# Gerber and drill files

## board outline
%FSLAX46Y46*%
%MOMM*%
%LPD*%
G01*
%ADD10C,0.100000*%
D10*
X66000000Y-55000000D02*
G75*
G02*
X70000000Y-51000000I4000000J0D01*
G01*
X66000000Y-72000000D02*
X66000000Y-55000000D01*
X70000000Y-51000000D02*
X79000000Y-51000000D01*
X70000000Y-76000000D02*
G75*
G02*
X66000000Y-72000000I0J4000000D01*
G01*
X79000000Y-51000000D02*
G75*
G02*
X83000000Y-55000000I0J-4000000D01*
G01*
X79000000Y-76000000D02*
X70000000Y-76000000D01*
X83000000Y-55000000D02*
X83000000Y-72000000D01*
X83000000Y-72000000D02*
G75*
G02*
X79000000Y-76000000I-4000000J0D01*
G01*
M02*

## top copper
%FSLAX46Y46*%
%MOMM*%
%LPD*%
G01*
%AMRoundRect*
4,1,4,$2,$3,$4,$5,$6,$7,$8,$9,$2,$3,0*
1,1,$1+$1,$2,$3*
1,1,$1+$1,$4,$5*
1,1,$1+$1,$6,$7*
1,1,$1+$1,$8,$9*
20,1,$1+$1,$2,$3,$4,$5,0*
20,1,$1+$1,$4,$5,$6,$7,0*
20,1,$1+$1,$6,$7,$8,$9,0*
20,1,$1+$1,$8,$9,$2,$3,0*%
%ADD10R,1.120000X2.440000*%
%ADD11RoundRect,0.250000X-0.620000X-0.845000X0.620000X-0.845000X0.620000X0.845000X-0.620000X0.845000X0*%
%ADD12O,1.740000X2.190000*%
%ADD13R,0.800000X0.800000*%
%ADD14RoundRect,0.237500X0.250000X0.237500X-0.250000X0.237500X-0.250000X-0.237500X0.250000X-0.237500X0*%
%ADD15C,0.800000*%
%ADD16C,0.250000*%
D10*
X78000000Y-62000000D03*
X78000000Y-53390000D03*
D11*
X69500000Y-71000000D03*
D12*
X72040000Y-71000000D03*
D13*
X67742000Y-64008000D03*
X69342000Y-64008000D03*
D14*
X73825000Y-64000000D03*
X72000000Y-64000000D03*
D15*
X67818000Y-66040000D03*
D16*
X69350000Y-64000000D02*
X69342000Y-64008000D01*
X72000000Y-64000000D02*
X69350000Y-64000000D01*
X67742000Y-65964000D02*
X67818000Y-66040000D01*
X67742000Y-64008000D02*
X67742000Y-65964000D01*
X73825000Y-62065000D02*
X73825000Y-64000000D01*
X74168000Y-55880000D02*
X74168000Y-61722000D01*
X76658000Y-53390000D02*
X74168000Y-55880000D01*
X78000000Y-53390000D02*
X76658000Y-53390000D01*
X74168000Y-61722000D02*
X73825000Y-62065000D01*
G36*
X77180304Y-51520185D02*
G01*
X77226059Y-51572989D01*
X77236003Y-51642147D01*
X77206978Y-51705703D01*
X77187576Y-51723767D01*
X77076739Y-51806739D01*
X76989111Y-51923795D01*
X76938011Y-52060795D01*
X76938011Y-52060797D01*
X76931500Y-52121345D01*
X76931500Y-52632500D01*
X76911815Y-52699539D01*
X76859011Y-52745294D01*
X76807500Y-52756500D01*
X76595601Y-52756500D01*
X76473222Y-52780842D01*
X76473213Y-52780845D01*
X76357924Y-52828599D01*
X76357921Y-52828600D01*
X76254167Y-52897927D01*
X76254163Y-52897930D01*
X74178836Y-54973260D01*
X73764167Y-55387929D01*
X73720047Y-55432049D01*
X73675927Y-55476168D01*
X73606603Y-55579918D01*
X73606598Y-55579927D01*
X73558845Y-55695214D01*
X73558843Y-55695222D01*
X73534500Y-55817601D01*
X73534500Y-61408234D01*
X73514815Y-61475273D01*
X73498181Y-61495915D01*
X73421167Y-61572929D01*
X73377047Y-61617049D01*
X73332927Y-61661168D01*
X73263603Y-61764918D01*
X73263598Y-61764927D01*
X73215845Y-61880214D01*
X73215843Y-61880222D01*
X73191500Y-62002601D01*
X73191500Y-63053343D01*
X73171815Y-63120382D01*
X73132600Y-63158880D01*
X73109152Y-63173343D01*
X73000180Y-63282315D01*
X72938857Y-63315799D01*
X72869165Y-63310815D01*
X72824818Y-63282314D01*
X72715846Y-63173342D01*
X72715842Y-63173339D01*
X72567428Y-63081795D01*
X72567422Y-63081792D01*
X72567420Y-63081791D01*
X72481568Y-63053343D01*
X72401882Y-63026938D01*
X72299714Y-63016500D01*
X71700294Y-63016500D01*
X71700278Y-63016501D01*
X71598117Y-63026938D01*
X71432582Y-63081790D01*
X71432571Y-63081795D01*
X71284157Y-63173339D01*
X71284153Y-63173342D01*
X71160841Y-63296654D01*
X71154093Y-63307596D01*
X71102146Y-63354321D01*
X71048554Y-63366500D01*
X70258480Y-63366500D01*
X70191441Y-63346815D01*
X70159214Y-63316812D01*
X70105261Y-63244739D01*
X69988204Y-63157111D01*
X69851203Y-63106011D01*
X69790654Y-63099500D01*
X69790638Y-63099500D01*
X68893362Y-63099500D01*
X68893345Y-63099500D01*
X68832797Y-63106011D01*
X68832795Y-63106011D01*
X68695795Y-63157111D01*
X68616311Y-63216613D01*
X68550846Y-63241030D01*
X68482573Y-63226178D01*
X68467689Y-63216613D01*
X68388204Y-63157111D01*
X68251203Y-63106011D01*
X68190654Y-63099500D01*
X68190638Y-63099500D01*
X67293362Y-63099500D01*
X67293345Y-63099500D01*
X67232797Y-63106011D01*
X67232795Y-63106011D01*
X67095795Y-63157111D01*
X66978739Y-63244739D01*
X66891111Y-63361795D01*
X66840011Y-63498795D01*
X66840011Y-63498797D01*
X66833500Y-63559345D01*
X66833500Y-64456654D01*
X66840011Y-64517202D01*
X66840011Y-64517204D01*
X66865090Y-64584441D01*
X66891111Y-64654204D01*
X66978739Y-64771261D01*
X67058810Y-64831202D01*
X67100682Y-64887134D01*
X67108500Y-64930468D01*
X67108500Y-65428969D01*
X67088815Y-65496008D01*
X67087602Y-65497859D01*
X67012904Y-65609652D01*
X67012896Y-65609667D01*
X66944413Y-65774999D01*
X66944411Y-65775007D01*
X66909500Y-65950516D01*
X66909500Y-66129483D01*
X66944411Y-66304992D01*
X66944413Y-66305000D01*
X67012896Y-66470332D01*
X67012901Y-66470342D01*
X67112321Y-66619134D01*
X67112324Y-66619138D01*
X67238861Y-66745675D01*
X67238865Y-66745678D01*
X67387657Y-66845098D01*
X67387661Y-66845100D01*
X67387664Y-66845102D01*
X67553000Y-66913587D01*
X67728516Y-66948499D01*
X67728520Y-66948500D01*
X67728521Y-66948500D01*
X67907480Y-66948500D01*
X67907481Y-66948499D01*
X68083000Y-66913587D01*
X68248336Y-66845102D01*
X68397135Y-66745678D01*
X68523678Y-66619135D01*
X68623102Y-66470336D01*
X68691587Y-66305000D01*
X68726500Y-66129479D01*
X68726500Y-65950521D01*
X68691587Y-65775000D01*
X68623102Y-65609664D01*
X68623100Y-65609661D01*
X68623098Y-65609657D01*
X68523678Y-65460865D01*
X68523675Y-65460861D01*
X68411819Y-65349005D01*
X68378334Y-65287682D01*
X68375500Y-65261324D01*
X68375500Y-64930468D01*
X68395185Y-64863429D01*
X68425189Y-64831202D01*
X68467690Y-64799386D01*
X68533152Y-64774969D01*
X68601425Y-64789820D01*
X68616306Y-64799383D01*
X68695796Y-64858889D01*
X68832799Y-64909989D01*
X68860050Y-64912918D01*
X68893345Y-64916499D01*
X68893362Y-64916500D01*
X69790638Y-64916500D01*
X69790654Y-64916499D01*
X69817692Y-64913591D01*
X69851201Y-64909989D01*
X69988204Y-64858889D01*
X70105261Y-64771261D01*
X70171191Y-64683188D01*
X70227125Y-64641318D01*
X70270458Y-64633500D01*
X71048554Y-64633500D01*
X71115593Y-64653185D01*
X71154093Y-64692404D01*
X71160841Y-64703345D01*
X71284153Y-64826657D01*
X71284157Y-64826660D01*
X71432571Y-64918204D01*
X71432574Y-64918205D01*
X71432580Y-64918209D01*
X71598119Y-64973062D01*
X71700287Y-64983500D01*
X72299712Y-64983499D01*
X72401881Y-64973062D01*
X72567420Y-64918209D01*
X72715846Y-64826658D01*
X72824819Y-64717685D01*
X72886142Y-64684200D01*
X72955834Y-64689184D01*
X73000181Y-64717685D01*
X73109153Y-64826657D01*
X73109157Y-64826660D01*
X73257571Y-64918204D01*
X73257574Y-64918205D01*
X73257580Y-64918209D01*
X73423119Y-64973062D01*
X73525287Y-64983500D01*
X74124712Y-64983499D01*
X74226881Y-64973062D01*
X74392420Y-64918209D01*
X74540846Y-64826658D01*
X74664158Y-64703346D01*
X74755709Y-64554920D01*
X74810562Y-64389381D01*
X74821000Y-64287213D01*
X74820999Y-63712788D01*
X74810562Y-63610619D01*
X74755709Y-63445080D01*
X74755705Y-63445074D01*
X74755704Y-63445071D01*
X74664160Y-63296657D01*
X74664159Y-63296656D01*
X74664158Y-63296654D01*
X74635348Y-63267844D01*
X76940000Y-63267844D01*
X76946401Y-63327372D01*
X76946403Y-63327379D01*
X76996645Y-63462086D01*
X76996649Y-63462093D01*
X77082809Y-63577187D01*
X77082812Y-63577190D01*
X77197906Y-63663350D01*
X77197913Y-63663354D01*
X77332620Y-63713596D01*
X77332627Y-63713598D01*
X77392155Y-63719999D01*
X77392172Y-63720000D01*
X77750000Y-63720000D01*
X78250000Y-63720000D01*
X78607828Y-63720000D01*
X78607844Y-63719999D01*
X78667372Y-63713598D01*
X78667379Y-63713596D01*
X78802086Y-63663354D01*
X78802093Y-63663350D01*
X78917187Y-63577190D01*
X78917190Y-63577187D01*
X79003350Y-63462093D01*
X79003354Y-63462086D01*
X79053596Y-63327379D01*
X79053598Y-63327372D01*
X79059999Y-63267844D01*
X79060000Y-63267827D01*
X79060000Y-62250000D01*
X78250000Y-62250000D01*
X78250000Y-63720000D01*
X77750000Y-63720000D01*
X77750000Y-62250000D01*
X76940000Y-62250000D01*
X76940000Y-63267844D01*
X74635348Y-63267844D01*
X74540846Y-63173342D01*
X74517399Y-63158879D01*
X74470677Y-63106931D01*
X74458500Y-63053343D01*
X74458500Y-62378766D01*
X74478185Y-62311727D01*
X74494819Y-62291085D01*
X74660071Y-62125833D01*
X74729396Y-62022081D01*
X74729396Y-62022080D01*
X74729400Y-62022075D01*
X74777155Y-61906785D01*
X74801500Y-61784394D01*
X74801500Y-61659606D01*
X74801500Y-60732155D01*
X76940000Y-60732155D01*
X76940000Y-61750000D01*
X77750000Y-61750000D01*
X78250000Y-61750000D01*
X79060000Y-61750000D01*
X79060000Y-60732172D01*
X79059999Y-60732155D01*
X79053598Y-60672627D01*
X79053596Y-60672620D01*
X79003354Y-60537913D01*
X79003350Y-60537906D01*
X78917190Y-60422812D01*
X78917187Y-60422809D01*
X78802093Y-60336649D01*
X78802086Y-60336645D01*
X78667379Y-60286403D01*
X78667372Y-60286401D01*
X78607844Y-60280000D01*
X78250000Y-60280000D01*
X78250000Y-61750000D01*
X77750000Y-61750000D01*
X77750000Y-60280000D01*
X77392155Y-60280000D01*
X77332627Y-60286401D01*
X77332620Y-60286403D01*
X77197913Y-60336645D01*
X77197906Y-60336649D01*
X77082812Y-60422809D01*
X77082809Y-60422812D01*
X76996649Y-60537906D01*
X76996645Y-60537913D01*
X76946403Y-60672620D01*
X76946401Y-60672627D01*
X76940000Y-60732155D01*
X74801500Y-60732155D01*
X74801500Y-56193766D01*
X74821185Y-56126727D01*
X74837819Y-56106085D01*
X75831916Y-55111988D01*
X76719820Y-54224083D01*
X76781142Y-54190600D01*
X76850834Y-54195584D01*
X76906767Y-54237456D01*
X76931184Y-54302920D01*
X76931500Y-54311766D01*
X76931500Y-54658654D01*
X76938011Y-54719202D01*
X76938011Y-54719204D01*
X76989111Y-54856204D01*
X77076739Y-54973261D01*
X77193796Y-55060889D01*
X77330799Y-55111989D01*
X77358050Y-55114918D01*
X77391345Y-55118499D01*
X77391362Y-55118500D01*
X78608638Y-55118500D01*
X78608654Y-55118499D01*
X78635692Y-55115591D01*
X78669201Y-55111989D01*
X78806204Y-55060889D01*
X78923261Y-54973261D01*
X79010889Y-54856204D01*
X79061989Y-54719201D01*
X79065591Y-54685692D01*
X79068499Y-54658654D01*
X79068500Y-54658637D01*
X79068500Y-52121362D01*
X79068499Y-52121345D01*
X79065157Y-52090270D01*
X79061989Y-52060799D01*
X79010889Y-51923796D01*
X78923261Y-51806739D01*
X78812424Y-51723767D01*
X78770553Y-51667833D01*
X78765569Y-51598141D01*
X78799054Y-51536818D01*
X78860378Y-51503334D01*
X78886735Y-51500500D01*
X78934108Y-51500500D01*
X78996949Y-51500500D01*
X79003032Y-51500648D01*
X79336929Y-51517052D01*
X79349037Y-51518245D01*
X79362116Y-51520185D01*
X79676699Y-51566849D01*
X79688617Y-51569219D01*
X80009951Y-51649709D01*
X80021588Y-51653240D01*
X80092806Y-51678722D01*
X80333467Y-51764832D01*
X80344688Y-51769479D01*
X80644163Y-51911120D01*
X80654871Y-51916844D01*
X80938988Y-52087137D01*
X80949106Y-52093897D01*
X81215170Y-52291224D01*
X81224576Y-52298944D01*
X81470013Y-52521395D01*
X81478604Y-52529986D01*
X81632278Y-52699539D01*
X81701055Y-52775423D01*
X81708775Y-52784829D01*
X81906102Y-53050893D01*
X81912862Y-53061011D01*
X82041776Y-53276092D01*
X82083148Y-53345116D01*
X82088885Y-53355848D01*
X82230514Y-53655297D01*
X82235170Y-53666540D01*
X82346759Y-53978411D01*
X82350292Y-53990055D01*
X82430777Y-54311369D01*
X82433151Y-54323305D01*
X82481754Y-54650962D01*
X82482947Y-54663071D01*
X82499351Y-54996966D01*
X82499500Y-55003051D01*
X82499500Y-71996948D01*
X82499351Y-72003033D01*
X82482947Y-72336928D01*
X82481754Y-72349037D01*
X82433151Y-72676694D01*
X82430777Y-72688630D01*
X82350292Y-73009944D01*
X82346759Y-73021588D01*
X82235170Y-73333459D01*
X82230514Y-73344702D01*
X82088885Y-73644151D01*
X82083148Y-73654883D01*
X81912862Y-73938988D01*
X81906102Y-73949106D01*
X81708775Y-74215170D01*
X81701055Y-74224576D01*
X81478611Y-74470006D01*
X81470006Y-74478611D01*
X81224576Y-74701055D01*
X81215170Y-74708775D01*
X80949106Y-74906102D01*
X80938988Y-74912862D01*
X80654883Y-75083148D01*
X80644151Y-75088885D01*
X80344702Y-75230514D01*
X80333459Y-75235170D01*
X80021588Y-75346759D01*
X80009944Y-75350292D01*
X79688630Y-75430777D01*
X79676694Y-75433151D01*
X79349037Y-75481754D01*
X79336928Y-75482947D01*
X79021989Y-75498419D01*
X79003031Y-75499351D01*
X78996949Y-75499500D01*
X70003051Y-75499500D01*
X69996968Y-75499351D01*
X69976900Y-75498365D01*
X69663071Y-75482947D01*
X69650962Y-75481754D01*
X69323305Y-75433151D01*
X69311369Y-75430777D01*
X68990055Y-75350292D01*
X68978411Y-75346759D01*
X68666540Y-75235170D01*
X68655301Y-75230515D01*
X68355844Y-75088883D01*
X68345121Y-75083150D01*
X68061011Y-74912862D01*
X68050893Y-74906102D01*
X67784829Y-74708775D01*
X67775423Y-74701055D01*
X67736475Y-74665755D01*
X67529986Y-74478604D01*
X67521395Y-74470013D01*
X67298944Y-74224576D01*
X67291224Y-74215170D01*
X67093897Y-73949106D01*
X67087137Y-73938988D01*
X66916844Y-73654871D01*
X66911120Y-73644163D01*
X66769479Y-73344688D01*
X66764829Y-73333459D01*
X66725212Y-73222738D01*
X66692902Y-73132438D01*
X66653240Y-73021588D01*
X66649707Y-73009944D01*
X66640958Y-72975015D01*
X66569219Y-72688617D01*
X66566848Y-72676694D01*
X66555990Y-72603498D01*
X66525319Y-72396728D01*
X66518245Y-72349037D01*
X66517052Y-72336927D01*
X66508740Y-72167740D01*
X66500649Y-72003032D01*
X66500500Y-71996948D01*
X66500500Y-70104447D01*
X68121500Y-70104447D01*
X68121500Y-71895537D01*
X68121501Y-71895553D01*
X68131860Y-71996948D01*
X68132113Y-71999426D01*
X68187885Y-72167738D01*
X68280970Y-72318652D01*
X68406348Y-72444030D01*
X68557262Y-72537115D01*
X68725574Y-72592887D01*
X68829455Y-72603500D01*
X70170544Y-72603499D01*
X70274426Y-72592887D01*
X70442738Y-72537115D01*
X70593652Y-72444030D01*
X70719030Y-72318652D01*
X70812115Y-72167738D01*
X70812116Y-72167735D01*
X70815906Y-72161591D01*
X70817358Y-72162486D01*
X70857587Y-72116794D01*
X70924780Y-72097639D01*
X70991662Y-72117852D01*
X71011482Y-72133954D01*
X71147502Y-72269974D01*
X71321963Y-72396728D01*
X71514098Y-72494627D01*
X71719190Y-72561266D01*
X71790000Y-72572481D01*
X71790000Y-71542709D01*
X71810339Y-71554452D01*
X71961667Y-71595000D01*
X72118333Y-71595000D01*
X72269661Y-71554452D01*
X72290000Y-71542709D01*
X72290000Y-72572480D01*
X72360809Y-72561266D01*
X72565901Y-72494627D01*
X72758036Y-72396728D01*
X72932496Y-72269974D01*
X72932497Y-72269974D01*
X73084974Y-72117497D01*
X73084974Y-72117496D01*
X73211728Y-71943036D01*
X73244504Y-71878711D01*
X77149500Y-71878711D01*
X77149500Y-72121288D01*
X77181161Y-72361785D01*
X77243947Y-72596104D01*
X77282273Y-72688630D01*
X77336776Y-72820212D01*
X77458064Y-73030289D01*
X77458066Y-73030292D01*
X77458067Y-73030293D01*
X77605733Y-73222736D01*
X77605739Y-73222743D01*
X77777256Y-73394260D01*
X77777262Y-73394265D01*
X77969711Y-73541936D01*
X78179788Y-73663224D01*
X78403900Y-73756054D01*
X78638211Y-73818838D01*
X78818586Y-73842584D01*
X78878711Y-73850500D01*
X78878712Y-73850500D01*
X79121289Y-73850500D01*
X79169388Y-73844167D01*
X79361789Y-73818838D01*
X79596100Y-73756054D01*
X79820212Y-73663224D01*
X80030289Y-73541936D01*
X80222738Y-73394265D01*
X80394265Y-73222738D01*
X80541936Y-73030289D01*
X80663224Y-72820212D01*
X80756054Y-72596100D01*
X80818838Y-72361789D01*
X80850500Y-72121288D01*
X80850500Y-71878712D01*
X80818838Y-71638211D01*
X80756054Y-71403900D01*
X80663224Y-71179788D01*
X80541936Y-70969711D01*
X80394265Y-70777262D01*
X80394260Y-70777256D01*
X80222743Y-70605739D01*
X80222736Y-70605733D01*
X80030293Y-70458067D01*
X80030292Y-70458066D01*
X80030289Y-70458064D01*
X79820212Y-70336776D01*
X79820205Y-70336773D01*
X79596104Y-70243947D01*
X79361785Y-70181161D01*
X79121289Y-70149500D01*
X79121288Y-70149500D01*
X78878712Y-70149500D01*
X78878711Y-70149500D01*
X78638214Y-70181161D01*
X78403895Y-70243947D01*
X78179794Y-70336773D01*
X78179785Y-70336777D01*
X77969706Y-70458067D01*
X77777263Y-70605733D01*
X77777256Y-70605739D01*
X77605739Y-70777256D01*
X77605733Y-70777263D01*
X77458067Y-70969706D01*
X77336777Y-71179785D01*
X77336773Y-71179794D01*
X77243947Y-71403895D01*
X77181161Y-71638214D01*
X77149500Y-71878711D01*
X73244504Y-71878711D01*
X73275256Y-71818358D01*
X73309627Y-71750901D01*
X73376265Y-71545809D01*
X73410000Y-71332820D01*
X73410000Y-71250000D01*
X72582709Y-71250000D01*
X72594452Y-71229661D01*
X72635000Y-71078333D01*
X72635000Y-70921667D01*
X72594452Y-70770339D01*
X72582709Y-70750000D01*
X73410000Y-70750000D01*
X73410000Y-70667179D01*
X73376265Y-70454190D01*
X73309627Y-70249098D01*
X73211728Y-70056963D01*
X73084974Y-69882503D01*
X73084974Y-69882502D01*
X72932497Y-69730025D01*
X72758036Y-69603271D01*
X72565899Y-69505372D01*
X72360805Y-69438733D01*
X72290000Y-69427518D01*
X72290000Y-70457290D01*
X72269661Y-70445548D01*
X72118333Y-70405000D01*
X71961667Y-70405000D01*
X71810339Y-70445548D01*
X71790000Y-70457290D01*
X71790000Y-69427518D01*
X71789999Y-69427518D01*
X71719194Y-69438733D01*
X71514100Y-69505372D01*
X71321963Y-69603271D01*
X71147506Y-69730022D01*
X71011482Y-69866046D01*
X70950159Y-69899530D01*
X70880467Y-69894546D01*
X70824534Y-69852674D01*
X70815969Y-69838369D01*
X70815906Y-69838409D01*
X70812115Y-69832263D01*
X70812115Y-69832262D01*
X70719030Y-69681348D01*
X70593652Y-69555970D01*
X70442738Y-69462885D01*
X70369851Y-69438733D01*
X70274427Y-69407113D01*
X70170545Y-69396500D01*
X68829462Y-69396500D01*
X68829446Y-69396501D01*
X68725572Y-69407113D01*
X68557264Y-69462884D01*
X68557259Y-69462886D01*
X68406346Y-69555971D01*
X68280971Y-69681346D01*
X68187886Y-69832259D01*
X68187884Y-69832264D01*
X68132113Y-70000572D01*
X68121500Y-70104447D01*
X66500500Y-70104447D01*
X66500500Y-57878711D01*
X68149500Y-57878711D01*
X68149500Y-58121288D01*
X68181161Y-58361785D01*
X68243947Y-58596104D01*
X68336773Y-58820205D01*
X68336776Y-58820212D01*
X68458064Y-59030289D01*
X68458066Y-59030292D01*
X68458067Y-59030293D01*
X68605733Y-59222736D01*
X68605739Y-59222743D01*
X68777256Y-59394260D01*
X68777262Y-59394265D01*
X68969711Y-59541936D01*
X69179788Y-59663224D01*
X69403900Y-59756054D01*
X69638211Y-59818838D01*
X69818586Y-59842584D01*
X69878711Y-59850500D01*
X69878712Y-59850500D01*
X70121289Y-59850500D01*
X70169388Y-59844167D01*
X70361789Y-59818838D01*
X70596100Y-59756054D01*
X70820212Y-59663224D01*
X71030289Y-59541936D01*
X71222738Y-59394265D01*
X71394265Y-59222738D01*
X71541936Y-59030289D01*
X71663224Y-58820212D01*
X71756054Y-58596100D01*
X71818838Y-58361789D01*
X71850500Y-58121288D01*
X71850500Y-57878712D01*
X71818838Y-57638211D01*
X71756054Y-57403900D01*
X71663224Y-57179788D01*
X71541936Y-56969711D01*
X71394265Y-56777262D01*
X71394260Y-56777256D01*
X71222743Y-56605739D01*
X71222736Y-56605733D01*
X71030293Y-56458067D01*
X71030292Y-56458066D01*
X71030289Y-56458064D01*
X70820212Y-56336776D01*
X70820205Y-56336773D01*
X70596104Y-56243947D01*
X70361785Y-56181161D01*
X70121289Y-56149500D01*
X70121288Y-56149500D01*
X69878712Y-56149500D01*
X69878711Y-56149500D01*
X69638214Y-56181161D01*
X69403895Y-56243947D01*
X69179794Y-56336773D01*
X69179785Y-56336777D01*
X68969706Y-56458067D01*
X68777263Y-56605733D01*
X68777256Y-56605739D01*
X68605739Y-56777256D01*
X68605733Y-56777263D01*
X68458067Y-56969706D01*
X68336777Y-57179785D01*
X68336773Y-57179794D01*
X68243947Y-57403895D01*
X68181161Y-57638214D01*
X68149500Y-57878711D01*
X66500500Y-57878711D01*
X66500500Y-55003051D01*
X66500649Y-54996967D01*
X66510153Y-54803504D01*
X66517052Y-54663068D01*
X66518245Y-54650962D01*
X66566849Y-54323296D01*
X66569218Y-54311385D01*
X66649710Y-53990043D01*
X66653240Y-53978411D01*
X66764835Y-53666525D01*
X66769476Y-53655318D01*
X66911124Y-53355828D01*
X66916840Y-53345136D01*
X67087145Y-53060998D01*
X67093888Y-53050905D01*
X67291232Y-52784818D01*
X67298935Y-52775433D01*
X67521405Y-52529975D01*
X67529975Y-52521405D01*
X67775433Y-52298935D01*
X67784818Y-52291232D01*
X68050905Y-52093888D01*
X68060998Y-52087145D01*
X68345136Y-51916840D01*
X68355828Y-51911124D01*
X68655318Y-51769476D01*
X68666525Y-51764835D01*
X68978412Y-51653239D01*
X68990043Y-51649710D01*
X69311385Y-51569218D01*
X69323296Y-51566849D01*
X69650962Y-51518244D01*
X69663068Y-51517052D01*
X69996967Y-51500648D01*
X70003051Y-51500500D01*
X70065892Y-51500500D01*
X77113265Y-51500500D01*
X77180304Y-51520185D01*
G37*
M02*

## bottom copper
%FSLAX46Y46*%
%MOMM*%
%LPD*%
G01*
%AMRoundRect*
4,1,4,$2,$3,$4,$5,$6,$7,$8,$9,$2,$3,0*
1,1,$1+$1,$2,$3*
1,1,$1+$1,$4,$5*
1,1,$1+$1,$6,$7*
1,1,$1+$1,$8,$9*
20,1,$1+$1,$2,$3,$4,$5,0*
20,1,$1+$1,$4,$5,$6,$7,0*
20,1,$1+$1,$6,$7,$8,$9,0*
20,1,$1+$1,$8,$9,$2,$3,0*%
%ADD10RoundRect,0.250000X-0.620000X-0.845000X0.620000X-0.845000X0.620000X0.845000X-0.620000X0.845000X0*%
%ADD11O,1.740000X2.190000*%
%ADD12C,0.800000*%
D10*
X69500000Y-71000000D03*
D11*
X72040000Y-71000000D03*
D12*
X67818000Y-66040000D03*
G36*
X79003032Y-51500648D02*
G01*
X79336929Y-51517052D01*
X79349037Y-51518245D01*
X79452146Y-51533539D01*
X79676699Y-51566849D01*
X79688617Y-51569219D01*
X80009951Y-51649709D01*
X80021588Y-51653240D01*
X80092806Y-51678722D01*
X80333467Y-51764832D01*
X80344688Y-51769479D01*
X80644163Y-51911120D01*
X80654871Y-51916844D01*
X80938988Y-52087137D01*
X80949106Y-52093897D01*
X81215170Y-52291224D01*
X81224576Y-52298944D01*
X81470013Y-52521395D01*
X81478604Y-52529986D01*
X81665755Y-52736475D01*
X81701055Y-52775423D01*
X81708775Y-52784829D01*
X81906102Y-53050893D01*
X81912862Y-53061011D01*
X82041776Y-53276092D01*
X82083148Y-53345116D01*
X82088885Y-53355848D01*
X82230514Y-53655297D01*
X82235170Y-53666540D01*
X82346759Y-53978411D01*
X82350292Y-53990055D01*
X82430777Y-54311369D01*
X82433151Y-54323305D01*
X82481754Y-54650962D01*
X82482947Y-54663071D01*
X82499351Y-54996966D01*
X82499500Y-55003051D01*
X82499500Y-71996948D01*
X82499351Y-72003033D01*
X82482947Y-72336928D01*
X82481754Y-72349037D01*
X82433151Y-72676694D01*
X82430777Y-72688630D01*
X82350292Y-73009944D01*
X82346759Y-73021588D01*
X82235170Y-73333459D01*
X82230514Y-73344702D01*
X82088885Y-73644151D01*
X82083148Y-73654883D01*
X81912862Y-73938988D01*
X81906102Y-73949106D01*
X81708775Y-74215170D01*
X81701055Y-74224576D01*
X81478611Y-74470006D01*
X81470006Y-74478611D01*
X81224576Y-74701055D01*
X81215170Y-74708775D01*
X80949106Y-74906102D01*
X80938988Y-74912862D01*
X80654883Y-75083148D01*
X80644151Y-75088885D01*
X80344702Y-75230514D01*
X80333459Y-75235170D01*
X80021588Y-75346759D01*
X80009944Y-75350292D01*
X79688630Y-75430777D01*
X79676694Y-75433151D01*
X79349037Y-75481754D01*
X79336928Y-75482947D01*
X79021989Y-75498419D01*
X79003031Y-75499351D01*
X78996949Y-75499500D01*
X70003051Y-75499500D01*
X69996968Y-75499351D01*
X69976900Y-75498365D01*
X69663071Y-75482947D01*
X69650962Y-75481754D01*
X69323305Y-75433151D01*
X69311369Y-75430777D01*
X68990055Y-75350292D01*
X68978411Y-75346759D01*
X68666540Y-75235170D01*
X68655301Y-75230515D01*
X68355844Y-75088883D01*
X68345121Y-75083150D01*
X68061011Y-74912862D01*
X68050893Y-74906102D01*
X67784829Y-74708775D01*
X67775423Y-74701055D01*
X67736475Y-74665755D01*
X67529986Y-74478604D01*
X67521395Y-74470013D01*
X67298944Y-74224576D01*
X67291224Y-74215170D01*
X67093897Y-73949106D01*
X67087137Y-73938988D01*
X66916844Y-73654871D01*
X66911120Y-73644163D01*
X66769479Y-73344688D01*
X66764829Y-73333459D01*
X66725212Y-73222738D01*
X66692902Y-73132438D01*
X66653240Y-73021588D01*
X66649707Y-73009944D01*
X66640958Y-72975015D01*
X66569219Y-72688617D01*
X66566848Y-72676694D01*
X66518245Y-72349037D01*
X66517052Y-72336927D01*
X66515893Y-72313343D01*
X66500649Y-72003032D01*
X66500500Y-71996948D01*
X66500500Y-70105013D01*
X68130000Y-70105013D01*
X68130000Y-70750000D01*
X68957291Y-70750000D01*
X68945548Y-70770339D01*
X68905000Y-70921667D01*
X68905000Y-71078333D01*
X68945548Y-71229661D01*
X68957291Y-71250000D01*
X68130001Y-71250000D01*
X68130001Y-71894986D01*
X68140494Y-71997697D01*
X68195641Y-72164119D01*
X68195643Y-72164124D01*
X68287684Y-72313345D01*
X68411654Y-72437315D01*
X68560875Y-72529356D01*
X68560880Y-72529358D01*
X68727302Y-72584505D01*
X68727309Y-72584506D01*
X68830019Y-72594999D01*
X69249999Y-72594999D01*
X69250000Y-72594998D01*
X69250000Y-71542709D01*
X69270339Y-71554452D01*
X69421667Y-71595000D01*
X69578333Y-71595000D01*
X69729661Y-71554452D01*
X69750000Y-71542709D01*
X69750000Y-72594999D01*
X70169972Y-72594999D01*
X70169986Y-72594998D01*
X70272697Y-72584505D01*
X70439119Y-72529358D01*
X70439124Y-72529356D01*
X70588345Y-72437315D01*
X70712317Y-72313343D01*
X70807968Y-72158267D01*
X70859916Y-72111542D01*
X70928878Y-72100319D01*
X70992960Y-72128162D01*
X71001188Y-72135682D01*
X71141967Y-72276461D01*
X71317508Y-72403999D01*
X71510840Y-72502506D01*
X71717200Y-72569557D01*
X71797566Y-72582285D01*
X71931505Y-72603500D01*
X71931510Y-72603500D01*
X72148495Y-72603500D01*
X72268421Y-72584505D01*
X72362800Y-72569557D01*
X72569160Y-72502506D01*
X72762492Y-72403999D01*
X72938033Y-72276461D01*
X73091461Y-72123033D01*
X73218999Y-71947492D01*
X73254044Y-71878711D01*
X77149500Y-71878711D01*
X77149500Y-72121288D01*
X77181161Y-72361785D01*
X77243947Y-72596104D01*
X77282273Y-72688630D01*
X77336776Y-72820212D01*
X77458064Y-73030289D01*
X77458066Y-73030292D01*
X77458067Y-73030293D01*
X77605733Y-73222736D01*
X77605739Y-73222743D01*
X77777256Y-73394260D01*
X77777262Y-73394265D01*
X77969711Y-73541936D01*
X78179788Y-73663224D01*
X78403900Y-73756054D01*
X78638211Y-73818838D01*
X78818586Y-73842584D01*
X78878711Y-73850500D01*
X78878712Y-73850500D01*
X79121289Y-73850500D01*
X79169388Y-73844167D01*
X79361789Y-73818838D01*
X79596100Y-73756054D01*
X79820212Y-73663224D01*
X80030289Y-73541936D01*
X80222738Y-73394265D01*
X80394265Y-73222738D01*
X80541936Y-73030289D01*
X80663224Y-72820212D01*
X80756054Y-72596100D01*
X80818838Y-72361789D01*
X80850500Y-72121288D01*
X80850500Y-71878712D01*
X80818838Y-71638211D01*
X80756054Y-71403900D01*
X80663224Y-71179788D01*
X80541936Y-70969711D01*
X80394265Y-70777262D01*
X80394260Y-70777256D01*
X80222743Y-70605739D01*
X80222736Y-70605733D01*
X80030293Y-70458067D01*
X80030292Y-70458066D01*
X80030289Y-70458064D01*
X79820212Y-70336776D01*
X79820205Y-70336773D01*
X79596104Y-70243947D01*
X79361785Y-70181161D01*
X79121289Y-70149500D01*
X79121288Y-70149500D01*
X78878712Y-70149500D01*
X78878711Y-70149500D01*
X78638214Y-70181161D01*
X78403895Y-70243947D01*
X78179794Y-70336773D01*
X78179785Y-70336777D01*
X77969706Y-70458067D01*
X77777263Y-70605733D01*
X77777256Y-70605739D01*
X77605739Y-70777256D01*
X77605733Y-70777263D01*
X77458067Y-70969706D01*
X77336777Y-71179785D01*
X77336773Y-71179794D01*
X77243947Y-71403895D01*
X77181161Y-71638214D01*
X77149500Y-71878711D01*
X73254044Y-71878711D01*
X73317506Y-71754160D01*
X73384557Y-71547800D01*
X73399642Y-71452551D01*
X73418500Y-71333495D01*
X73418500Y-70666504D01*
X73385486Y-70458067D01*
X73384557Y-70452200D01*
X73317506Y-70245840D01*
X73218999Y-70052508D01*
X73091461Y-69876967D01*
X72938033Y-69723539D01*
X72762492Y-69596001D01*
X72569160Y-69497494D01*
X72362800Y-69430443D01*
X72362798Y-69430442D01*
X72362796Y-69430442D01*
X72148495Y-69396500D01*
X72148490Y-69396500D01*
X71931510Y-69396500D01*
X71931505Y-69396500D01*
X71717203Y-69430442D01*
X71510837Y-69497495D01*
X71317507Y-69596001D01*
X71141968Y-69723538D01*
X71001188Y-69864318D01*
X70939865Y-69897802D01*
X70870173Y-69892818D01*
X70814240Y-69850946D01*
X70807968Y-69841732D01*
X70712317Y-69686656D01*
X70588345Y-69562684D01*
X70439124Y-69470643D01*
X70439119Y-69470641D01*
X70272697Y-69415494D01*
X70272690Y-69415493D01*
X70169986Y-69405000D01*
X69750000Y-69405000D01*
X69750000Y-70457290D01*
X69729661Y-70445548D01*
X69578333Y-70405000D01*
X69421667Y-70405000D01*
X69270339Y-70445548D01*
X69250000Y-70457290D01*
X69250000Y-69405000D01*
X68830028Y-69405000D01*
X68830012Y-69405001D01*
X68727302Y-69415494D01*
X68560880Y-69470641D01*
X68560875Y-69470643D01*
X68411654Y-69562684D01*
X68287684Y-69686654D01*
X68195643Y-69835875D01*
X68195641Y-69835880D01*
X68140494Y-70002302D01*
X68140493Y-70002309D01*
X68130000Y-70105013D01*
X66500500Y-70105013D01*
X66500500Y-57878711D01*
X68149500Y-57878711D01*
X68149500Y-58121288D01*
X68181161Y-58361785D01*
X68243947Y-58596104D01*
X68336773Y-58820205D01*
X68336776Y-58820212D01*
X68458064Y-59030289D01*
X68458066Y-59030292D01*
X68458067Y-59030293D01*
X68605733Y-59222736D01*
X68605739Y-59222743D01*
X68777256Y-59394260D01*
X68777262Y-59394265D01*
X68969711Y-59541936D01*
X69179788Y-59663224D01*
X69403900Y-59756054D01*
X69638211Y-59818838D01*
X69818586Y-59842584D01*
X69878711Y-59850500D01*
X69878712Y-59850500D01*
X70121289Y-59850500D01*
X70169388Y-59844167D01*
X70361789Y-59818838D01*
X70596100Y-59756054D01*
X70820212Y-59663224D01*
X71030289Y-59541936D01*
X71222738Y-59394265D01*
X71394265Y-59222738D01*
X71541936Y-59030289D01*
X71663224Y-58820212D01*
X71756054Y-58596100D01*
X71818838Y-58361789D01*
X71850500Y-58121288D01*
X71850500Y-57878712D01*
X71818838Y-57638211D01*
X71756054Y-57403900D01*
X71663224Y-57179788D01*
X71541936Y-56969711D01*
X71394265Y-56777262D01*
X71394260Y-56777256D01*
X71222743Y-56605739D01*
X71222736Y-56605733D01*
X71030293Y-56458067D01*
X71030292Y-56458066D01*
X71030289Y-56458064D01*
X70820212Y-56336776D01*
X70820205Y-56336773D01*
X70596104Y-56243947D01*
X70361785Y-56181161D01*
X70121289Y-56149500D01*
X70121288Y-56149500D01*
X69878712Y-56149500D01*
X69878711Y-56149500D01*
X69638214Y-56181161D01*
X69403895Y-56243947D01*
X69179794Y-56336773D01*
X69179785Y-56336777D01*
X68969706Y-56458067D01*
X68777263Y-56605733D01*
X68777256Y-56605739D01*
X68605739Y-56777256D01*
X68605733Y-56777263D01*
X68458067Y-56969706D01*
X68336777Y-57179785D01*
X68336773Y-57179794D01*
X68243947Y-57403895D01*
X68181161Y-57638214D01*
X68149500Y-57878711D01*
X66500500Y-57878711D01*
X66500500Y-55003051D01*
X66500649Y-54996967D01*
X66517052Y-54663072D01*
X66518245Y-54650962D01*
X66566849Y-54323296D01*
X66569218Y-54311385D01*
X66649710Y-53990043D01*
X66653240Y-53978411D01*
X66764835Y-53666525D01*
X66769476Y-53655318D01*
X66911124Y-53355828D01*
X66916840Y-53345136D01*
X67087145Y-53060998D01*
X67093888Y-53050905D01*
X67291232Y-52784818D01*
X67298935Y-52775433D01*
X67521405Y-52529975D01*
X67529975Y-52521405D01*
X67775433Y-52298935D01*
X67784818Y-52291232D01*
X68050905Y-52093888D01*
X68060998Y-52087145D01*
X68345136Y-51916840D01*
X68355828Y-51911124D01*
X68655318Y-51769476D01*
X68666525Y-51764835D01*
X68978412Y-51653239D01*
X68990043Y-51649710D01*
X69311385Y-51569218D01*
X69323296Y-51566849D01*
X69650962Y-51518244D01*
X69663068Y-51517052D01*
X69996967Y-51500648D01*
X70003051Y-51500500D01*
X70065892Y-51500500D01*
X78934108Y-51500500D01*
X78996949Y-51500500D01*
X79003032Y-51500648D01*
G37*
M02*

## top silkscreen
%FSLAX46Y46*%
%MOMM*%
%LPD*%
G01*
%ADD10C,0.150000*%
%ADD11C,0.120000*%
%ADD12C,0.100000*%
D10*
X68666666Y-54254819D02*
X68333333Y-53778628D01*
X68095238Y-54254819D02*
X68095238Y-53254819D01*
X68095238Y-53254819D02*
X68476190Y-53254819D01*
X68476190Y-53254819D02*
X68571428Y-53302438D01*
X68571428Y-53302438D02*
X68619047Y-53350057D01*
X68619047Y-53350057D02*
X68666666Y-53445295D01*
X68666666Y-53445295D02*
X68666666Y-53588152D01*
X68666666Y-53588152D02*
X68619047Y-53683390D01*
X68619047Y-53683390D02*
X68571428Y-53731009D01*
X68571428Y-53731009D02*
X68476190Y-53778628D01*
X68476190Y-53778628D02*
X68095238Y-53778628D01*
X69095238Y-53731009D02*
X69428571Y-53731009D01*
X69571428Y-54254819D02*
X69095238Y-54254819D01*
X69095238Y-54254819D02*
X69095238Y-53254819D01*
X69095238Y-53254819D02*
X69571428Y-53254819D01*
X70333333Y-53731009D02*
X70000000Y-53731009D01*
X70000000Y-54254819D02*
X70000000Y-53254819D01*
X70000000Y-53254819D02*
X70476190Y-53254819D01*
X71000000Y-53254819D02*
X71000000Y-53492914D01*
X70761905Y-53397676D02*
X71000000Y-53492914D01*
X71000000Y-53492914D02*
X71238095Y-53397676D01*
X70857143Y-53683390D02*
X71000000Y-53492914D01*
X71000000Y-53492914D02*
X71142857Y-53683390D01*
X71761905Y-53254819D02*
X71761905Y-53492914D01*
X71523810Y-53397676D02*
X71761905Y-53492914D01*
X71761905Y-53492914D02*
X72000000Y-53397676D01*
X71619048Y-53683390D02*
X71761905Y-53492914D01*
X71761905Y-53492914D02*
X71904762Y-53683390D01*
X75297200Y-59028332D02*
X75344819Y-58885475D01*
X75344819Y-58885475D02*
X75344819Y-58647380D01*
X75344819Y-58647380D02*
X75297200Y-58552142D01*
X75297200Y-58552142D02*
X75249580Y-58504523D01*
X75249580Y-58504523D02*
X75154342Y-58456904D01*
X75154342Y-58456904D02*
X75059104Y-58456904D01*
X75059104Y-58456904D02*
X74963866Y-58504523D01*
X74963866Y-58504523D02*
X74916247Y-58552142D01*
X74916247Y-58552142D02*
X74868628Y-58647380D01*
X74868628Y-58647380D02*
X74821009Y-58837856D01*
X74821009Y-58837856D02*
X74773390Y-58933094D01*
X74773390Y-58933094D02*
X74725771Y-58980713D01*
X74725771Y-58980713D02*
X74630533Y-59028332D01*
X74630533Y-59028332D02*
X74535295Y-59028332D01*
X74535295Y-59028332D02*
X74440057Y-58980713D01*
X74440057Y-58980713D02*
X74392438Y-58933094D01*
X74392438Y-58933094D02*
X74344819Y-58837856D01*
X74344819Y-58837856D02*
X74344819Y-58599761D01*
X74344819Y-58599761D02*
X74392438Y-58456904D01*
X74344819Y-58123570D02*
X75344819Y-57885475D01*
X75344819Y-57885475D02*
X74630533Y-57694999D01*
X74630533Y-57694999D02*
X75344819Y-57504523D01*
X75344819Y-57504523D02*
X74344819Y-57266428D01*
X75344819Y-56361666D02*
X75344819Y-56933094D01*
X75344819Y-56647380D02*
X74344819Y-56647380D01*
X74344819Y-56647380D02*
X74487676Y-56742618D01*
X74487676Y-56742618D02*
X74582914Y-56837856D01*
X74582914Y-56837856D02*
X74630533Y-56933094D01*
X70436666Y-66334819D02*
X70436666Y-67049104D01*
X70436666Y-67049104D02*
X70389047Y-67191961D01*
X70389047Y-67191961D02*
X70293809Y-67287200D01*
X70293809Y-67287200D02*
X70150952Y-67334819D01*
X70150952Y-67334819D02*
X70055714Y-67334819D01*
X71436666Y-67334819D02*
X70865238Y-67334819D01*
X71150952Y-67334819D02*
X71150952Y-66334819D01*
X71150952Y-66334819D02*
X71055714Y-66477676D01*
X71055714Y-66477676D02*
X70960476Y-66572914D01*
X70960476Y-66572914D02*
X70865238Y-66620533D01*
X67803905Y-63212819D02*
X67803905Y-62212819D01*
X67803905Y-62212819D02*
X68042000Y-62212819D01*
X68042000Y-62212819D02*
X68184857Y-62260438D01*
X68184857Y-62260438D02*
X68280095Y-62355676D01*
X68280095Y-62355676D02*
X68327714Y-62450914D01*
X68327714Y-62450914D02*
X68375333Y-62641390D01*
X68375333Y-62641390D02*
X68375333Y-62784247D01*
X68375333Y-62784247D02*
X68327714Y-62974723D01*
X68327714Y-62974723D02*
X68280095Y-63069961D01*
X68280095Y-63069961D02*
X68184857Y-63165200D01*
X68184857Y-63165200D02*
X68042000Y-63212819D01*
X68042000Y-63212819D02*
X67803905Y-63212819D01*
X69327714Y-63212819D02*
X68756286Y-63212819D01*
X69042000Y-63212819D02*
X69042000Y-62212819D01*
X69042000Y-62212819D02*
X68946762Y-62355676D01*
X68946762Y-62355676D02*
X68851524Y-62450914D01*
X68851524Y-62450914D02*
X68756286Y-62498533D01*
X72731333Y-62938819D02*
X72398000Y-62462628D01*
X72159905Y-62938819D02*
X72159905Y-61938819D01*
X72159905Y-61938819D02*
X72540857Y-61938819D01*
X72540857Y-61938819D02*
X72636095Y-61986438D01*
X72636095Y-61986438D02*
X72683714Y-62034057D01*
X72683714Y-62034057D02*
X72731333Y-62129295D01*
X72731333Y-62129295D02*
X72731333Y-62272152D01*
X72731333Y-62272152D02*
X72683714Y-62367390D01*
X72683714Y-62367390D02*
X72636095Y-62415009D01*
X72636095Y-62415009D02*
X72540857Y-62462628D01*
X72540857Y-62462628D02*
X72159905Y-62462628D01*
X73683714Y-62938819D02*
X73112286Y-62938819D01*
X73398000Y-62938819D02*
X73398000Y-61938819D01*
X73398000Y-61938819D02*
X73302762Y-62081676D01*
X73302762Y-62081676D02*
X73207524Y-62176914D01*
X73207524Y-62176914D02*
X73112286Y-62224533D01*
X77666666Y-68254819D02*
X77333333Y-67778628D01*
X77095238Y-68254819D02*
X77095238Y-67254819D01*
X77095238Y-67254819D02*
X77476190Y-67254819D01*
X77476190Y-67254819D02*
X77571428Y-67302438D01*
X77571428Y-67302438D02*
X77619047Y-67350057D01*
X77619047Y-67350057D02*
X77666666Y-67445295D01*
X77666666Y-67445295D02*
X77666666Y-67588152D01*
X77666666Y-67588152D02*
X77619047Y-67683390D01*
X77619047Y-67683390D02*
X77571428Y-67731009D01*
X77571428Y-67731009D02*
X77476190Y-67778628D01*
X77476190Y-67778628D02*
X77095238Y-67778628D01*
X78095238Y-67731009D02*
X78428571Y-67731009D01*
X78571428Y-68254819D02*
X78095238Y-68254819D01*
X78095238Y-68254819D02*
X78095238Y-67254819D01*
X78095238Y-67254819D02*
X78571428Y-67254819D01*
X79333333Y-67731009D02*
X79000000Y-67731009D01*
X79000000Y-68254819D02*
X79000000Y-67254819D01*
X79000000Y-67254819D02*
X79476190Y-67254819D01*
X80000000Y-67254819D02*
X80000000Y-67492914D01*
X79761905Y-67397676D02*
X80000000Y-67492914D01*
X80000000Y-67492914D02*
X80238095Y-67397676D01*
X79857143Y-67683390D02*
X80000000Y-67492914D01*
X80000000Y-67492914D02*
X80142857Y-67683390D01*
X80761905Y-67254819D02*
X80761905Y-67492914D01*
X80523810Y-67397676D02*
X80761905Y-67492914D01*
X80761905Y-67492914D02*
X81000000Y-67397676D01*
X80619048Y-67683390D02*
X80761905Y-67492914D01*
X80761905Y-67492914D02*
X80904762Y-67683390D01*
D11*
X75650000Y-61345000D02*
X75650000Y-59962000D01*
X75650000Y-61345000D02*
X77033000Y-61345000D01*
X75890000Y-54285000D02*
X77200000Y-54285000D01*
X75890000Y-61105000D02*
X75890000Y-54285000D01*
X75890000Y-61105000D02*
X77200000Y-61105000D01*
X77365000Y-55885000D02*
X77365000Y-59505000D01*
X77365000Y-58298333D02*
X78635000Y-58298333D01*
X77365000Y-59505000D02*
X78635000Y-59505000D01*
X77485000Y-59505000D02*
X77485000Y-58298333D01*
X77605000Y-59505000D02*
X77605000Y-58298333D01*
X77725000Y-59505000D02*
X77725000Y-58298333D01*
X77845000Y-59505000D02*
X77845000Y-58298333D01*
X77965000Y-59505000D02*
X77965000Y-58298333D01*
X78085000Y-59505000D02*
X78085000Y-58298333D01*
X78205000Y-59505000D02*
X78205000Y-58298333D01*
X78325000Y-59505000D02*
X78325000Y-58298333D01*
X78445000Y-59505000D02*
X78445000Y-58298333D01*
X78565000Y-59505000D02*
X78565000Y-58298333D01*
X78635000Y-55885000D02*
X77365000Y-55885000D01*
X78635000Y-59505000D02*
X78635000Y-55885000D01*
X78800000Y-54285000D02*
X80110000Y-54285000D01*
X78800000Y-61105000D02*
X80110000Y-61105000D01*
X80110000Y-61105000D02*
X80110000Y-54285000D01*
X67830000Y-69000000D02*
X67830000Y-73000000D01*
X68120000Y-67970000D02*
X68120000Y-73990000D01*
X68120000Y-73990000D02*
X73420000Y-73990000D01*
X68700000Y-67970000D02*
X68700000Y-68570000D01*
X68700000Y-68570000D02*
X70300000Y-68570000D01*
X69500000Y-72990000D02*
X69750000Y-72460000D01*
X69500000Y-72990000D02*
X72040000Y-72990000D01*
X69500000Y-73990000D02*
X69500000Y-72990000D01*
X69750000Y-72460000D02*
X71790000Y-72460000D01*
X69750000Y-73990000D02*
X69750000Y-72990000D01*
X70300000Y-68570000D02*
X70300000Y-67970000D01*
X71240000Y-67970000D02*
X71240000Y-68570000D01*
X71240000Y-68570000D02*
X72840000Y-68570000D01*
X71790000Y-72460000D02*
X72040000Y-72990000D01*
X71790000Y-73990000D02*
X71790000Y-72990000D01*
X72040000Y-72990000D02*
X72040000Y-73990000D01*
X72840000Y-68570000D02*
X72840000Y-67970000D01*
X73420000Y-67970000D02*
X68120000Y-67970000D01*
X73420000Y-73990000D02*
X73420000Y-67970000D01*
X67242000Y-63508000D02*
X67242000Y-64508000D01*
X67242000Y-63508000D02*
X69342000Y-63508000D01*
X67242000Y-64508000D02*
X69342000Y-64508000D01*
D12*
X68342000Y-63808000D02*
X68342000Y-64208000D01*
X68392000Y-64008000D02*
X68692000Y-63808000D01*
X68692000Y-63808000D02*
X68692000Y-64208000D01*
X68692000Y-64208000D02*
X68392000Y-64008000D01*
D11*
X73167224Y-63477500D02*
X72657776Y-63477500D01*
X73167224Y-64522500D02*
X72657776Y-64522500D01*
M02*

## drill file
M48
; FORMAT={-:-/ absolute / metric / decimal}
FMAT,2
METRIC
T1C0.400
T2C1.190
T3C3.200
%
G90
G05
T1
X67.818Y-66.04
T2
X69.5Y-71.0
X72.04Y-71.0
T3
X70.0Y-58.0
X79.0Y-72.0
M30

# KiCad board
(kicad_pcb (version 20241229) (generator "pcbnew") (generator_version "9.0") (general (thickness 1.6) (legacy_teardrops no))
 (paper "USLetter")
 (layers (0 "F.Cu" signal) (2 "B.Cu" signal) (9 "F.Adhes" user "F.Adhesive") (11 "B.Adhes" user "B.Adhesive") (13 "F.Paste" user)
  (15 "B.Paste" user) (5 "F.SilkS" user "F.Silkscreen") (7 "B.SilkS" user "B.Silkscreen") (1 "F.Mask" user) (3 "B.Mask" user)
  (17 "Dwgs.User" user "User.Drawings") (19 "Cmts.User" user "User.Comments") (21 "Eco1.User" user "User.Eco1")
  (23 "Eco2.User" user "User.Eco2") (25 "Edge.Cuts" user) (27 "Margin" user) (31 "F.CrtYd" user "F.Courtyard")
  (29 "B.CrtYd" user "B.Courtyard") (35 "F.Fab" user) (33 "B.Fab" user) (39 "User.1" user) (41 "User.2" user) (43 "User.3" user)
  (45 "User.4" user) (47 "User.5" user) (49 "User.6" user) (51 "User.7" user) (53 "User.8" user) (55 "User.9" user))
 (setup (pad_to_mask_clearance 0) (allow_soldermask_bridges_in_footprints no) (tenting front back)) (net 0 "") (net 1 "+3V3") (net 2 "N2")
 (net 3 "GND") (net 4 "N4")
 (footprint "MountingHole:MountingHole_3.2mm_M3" (layer "F.Cu") (at 70 58)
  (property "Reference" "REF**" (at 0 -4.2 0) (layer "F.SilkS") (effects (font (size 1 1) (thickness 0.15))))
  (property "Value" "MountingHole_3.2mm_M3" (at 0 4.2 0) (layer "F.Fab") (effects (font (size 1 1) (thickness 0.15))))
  (pad "" np_thru_hole circle (at 0 0) (size 3.2 3.2) (drill 3.2) (layers "*.Cu" "*.Mask")))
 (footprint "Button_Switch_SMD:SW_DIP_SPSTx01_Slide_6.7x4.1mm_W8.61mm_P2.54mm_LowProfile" (layer "F.Cu") (at 78 57.695 90)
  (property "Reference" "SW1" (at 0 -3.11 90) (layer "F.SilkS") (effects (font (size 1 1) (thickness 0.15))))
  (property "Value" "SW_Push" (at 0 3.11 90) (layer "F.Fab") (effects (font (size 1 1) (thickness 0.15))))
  (fp_line (start -3.65 -2.35) (end -2.267 -2.35) (stroke (width 0.12) (type solid)) (layer "F.SilkS"))
  (fp_line (start -3.65 -2.35) (end -3.65 -0.967) (stroke (width 0.12) (type solid)) (layer "F.SilkS"))
  (fp_line (start 3.41 -2.11) (end 3.41 -0.8) (stroke (width 0.12) (type solid)) (layer "F.SilkS"))
  (fp_line (start -3.41 -2.11) (end 3.41 -2.11) (stroke (width 0.12) (type solid)) (layer "F.SilkS"))
  (fp_line (start -3.41 -2.11) (end -3.41 -0.8) (stroke (width 0.12) (type solid)) (layer "F.SilkS"))
  (fp_line (start 1.81 -0.635) (end -1.81 -0.635) (stroke (width 0.12) (type solid)) (layer "F.SilkS"))
  (fp_line (start -0.603333 -0.635) (end -0.603333 0.635) (stroke (width 0.12) (type solid)) (layer "F.SilkS"))
  (fp_line (start -1.81 -0.635) (end -1.81 0.635) (stroke (width 0.12) (type solid)) (layer "F.SilkS"))
  (fp_line (start -1.81 -0.515) (end -0.603333 -0.515) (stroke (width 0.12) (type solid)) (layer "F.SilkS"))
  (fp_line (start -1.81 -0.395) (end -0.603333 -0.395) (stroke (width 0.12) (type solid)) (layer "F.SilkS"))
  (fp_line (start -1.81 -0.275) (end -0.603333 -0.275) (stroke (width 0.12) (type solid)) (layer "F.SilkS"))
  (fp_line (start -1.81 -0.155) (end -0.603333 -0.155) (stroke (width 0.12) (type solid)) (layer "F.SilkS"))
  (fp_line (start -1.81 -0.035) (end -0.603333 -0.035) (stroke (width 0.12) (type solid)) (layer "F.SilkS"))
  (fp_line (start -1.81 0.085) (end -0.603333 0.085) (stroke (width 0.12) (type solid)) (layer "F.SilkS"))
  (fp_line (start -1.81 0.205) (end -0.603333 0.205) (stroke (width 0.12) (type solid)) (layer "F.SilkS"))
  (fp_line (start -1.81 0.325) (end -0.603333 0.325) (stroke (width 0.12) (type solid)) (layer "F.SilkS"))
  (fp_line (start -1.81 0.445) (end -0.603333 0.445) (stroke (width 0.12) (type solid)) (layer "F.SilkS"))
  (fp_line (start -1.81 0.565) (end -0.603333 0.565) (stroke (width 0.12) (type solid)) (layer "F.SilkS"))
  (fp_line (start 1.81 0.635) (end 1.81 -0.635) (stroke (width 0.12) (type solid)) (layer "F.SilkS"))
  (fp_line (start -1.81 0.635) (end 1.81 0.635) (stroke (width 0.12) (type solid)) (layer "F.SilkS"))
  (fp_line (start 3.41 0.8) (end 3.41 2.11) (stroke (width 0.12) (type solid)) (layer "F.SilkS"))
  (fp_line (start -3.41 0.8) (end -3.41 2.11) (stroke (width 0.12) (type solid)) (layer "F.SilkS"))
  (fp_line (start -3.41 2.11) (end 3.41 2.11) (stroke (width 0.12) (type solid)) (layer "F.SilkS"))
  (pad "1" smd rect (at -4.305 0 90) (size 2.44 1.12) (layers "F.Cu" "F.Mask" "F.Paste") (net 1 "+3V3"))
  (pad "2" smd rect (at 4.305 0 90) (size 2.44 1.12) (layers "F.Cu" "F.Mask" "F.Paste") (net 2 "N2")))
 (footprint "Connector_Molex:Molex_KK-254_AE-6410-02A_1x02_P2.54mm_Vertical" (layer "F.Cu") (at 69.5 71)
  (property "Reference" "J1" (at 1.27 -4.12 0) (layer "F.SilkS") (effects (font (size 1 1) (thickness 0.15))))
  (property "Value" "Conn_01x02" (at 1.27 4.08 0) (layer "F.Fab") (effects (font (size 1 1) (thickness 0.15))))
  (fp_line (start -1.67 -2) (end -1.67 2) (stroke (width 0.12) (type solid)) (layer "F.SilkS"))
  (fp_line (start -1.38 -3.03) (end -1.38 2.99) (stroke (width 0.12) (type solid)) (layer "F.SilkS"))
  (fp_line (start -1.38 2.99) (end 3.92 2.99) (stroke (width 0.12) (type solid)) (layer "F.SilkS"))
  (fp_line (start -0.8 -3.03) (end -0.8 -2.43) (stroke (width 0.12) (type solid)) (layer "F.SilkS"))
  (fp_line (start -0.8 -2.43) (end 0.8 -2.43) (stroke (width 0.12) (type solid)) (layer "F.SilkS"))
  (fp_line (start 0 1.99) (end 0.25 1.46) (stroke (width 0.12) (type solid)) (layer "F.SilkS"))
  (fp_line (start 0 1.99) (end 2.54 1.99) (stroke (width 0.12) (type solid)) (layer "F.SilkS"))
  (fp_line (start 0 2.99) (end 0 1.99) (stroke (width 0.12) (type solid)) (layer "F.SilkS"))
  (fp_line (start 0.25 1.46) (end 2.29 1.46) (stroke (width 0.12) (type solid)) (layer "F.SilkS"))
  (fp_line (start 0.25 2.99) (end 0.25 1.99) (stroke (width 0.12) (type solid)) (layer "F.SilkS"))
  (fp_line (start 0.8 -2.43) (end 0.8 -3.03) (stroke (width 0.12) (type solid)) (layer "F.SilkS"))
  (fp_line (start 1.74 -3.03) (end 1.74 -2.43) (stroke (width 0.12) (type solid)) (layer "F.SilkS"))
  (fp_line (start 1.74 -2.43) (end 3.34 -2.43) (stroke (width 0.12) (type solid)) (layer "F.SilkS"))
  (fp_line (start 2.29 1.46) (end 2.54 1.99) (stroke (width 0.12) (type solid)) (layer "F.SilkS"))
  (fp_line (start 2.29 2.99) (end 2.29 1.99) (stroke (width 0.12) (type solid)) (layer "F.SilkS"))
  (fp_line (start 2.54 1.99) (end 2.54 2.99) (stroke (width 0.12) (type solid)) (layer "F.SilkS"))
  (fp_line (start 3.34 -2.43) (end 3.34 -3.03) (stroke (width 0.12) (type solid)) (layer "F.SilkS"))
  (fp_line (start 3.92 -3.03) (end -1.38 -3.03) (stroke (width 0.12) (type solid)) (layer "F.SilkS"))
  (fp_line (start 3.92 2.99) (end 3.92 -3.03) (stroke (width 0.12) (type solid)) (layer "F.SilkS"))
  (pad "1" thru_hole roundrect (at 0 0) (size 1.74 2.19) (drill 1.19) (layers "*.Cu" "*.Mask") (remove_unused_layers no)
   (roundrect_rratio 0.143678) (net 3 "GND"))
  (pad "2" thru_hole oval (at 2.54 0) (size 1.74 2.19) (drill 1.19) (layers "*.Cu" "*.Mask") (remove_unused_layers no) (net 1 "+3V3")))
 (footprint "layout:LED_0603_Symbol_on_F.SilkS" (layer "F.Cu") (at 68.542 64.008)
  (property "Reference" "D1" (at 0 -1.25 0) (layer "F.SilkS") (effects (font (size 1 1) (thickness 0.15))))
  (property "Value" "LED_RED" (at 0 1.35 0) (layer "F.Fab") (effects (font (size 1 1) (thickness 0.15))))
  (fp_line (start -1.3 -0.5) (end -1.3 0.5) (stroke (width 0.12) (type solid)) (layer "F.SilkS"))
  (fp_line (start -1.3 -0.5) (end 0.8 -0.5) (stroke (width 0.12) (type solid)) (layer "F.SilkS"))
  (fp_line (start -1.3 0.5) (end 0.8 0.5) (stroke (width 0.12) (type solid)) (layer "F.SilkS"))
  (fp_line (start -0.2 -0.2) (end -0.2 0.2) (stroke (width 0.1) (type solid)) (layer "F.SilkS"))
  (fp_line (start -0.15 0) (end 0.15 -0.2) (stroke (width 0.1) (type solid)) (layer "F.SilkS"))
  (fp_line (start 0.15 -0.2) (end 0.15 0.2) (stroke (width 0.1) (type solid)) (layer "F.SilkS"))
  (fp_line (start 0.15 0.2) (end -0.15 0) (stroke (width 0.1) (type solid)) (layer "F.SilkS"))
  (pad "1" smd rect (at -0.8 0 180) (size 0.8 0.8) (layers "F.Cu" "F.Mask" "F.Paste") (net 3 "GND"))
  (pad "2" smd rect (at 0.8 0 180) (size 0.8 0.8) (layers "F.Cu" "F.Mask" "F.Paste") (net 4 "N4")))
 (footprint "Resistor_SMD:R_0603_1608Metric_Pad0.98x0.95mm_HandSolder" (layer "F.Cu") (at 72.9125 64 180)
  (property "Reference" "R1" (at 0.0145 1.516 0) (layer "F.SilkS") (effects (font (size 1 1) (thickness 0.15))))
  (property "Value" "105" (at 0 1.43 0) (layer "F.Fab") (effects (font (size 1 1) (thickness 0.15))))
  (fp_line (start -0.254724 0.5225) (end 0.254724 0.5225) (stroke (width 0.12) (type solid)) (layer "F.SilkS"))
  (fp_line (start -0.254724 -0.5225) (end 0.254724 -0.5225) (stroke (width 0.12) (type solid)) (layer "F.SilkS"))
  (pad "1" smd roundrect (at -0.9125 0 180) (size 0.975 0.95) (layers "F.Cu" "F.Mask" "F.Paste") (roundrect_rratio 0.25) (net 2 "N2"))
  (pad "2" smd roundrect (at 0.9125 0 180) (size 0.975 0.95) (layers "F.Cu" "F.Mask" "F.Paste") (roundrect_rratio 0.25) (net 4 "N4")))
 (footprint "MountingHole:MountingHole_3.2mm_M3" (layer "F.Cu") (at 79 72)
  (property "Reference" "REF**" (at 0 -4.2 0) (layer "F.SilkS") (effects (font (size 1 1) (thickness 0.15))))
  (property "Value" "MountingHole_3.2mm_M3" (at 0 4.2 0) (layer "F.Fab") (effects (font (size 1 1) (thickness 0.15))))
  (pad "" np_thru_hole circle (at 0 0) (size 3.2 3.2) (drill 3.2) (layers "*.Cu" "*.Mask")))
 (gr_arc (start 66 55) (mid 67.171573 52.171573) (end 70 51) (stroke (width 0.1) (type default)) (layer "Edge.Cuts"))
 (gr_line (start 66 72) (end 66 55) (stroke (width 0.1) (type default)) (layer "Edge.Cuts"))
 (gr_line (start 70 51) (end 79 51) (stroke (width 0.1) (type default)) (layer "Edge.Cuts"))
 (gr_arc (start 70 76) (mid 67.171573 74.828427) (end 66 72) (stroke (width 0.1) (type default)) (layer "Edge.Cuts"))
 (gr_arc (start 79 51) (mid 81.828427 52.171573) (end 83 55) (stroke (width 0.1) (type default)) (layer "Edge.Cuts"))
 (gr_line (start 79 76) (end 70 76) (stroke (width 0.1) (type default)) (layer "Edge.Cuts"))
 (gr_line (start 83 55) (end 83 72) (stroke (width 0.1) (type default)) (layer "Edge.Cuts"))
 (gr_arc (start 83 72) (mid 81.828427 74.828427) (end 79 76) (stroke (width 0.1) (type default)) (layer "Edge.Cuts"))
 (segment (start 69.35 64) (end 69.342 64.008) (width 0.25) (layer "F.Cu") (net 4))
 (segment (start 72 64) (end 69.35 64) (width 0.25) (layer "F.Cu") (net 4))
 (segment (start 67.742 65.964) (end 67.818 66.04) (width 0.25) (layer "F.Cu") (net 3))
 (segment (start 67.742 64.008) (end 67.742 65.964) (width 0.25) (layer "F.Cu") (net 3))
 (via (at 67.818 66.04) (size 0.8) (drill 0.4) (layers "F.Cu" "B.Cu") (free yes) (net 3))
 (segment (start 73.825 62.065) (end 73.825 64) (width 0.25) (layer "F.Cu") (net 2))
 (segment (start 74.168 55.88) (end 74.168 61.722) (width 0.25) (layer "F.Cu") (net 2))
 (segment (start 76.658 53.39) (end 74.168 55.88) (width 0.25) (layer "F.Cu") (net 2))
 (segment (start 78 53.39) (end 76.658 53.39) (width 0.25) (layer "F.Cu") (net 2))
 (segment (start 74.168 61.722) (end 73.825 62.065) (width 0.25) (layer "F.Cu") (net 2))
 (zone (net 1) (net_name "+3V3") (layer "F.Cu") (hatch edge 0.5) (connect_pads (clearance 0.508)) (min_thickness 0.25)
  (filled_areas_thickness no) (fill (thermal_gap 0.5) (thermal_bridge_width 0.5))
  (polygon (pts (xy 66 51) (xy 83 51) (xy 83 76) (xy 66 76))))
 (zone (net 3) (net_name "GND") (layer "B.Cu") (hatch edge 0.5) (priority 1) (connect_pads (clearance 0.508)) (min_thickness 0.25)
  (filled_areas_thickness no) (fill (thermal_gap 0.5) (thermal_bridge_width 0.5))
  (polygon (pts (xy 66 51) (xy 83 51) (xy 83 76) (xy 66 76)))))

